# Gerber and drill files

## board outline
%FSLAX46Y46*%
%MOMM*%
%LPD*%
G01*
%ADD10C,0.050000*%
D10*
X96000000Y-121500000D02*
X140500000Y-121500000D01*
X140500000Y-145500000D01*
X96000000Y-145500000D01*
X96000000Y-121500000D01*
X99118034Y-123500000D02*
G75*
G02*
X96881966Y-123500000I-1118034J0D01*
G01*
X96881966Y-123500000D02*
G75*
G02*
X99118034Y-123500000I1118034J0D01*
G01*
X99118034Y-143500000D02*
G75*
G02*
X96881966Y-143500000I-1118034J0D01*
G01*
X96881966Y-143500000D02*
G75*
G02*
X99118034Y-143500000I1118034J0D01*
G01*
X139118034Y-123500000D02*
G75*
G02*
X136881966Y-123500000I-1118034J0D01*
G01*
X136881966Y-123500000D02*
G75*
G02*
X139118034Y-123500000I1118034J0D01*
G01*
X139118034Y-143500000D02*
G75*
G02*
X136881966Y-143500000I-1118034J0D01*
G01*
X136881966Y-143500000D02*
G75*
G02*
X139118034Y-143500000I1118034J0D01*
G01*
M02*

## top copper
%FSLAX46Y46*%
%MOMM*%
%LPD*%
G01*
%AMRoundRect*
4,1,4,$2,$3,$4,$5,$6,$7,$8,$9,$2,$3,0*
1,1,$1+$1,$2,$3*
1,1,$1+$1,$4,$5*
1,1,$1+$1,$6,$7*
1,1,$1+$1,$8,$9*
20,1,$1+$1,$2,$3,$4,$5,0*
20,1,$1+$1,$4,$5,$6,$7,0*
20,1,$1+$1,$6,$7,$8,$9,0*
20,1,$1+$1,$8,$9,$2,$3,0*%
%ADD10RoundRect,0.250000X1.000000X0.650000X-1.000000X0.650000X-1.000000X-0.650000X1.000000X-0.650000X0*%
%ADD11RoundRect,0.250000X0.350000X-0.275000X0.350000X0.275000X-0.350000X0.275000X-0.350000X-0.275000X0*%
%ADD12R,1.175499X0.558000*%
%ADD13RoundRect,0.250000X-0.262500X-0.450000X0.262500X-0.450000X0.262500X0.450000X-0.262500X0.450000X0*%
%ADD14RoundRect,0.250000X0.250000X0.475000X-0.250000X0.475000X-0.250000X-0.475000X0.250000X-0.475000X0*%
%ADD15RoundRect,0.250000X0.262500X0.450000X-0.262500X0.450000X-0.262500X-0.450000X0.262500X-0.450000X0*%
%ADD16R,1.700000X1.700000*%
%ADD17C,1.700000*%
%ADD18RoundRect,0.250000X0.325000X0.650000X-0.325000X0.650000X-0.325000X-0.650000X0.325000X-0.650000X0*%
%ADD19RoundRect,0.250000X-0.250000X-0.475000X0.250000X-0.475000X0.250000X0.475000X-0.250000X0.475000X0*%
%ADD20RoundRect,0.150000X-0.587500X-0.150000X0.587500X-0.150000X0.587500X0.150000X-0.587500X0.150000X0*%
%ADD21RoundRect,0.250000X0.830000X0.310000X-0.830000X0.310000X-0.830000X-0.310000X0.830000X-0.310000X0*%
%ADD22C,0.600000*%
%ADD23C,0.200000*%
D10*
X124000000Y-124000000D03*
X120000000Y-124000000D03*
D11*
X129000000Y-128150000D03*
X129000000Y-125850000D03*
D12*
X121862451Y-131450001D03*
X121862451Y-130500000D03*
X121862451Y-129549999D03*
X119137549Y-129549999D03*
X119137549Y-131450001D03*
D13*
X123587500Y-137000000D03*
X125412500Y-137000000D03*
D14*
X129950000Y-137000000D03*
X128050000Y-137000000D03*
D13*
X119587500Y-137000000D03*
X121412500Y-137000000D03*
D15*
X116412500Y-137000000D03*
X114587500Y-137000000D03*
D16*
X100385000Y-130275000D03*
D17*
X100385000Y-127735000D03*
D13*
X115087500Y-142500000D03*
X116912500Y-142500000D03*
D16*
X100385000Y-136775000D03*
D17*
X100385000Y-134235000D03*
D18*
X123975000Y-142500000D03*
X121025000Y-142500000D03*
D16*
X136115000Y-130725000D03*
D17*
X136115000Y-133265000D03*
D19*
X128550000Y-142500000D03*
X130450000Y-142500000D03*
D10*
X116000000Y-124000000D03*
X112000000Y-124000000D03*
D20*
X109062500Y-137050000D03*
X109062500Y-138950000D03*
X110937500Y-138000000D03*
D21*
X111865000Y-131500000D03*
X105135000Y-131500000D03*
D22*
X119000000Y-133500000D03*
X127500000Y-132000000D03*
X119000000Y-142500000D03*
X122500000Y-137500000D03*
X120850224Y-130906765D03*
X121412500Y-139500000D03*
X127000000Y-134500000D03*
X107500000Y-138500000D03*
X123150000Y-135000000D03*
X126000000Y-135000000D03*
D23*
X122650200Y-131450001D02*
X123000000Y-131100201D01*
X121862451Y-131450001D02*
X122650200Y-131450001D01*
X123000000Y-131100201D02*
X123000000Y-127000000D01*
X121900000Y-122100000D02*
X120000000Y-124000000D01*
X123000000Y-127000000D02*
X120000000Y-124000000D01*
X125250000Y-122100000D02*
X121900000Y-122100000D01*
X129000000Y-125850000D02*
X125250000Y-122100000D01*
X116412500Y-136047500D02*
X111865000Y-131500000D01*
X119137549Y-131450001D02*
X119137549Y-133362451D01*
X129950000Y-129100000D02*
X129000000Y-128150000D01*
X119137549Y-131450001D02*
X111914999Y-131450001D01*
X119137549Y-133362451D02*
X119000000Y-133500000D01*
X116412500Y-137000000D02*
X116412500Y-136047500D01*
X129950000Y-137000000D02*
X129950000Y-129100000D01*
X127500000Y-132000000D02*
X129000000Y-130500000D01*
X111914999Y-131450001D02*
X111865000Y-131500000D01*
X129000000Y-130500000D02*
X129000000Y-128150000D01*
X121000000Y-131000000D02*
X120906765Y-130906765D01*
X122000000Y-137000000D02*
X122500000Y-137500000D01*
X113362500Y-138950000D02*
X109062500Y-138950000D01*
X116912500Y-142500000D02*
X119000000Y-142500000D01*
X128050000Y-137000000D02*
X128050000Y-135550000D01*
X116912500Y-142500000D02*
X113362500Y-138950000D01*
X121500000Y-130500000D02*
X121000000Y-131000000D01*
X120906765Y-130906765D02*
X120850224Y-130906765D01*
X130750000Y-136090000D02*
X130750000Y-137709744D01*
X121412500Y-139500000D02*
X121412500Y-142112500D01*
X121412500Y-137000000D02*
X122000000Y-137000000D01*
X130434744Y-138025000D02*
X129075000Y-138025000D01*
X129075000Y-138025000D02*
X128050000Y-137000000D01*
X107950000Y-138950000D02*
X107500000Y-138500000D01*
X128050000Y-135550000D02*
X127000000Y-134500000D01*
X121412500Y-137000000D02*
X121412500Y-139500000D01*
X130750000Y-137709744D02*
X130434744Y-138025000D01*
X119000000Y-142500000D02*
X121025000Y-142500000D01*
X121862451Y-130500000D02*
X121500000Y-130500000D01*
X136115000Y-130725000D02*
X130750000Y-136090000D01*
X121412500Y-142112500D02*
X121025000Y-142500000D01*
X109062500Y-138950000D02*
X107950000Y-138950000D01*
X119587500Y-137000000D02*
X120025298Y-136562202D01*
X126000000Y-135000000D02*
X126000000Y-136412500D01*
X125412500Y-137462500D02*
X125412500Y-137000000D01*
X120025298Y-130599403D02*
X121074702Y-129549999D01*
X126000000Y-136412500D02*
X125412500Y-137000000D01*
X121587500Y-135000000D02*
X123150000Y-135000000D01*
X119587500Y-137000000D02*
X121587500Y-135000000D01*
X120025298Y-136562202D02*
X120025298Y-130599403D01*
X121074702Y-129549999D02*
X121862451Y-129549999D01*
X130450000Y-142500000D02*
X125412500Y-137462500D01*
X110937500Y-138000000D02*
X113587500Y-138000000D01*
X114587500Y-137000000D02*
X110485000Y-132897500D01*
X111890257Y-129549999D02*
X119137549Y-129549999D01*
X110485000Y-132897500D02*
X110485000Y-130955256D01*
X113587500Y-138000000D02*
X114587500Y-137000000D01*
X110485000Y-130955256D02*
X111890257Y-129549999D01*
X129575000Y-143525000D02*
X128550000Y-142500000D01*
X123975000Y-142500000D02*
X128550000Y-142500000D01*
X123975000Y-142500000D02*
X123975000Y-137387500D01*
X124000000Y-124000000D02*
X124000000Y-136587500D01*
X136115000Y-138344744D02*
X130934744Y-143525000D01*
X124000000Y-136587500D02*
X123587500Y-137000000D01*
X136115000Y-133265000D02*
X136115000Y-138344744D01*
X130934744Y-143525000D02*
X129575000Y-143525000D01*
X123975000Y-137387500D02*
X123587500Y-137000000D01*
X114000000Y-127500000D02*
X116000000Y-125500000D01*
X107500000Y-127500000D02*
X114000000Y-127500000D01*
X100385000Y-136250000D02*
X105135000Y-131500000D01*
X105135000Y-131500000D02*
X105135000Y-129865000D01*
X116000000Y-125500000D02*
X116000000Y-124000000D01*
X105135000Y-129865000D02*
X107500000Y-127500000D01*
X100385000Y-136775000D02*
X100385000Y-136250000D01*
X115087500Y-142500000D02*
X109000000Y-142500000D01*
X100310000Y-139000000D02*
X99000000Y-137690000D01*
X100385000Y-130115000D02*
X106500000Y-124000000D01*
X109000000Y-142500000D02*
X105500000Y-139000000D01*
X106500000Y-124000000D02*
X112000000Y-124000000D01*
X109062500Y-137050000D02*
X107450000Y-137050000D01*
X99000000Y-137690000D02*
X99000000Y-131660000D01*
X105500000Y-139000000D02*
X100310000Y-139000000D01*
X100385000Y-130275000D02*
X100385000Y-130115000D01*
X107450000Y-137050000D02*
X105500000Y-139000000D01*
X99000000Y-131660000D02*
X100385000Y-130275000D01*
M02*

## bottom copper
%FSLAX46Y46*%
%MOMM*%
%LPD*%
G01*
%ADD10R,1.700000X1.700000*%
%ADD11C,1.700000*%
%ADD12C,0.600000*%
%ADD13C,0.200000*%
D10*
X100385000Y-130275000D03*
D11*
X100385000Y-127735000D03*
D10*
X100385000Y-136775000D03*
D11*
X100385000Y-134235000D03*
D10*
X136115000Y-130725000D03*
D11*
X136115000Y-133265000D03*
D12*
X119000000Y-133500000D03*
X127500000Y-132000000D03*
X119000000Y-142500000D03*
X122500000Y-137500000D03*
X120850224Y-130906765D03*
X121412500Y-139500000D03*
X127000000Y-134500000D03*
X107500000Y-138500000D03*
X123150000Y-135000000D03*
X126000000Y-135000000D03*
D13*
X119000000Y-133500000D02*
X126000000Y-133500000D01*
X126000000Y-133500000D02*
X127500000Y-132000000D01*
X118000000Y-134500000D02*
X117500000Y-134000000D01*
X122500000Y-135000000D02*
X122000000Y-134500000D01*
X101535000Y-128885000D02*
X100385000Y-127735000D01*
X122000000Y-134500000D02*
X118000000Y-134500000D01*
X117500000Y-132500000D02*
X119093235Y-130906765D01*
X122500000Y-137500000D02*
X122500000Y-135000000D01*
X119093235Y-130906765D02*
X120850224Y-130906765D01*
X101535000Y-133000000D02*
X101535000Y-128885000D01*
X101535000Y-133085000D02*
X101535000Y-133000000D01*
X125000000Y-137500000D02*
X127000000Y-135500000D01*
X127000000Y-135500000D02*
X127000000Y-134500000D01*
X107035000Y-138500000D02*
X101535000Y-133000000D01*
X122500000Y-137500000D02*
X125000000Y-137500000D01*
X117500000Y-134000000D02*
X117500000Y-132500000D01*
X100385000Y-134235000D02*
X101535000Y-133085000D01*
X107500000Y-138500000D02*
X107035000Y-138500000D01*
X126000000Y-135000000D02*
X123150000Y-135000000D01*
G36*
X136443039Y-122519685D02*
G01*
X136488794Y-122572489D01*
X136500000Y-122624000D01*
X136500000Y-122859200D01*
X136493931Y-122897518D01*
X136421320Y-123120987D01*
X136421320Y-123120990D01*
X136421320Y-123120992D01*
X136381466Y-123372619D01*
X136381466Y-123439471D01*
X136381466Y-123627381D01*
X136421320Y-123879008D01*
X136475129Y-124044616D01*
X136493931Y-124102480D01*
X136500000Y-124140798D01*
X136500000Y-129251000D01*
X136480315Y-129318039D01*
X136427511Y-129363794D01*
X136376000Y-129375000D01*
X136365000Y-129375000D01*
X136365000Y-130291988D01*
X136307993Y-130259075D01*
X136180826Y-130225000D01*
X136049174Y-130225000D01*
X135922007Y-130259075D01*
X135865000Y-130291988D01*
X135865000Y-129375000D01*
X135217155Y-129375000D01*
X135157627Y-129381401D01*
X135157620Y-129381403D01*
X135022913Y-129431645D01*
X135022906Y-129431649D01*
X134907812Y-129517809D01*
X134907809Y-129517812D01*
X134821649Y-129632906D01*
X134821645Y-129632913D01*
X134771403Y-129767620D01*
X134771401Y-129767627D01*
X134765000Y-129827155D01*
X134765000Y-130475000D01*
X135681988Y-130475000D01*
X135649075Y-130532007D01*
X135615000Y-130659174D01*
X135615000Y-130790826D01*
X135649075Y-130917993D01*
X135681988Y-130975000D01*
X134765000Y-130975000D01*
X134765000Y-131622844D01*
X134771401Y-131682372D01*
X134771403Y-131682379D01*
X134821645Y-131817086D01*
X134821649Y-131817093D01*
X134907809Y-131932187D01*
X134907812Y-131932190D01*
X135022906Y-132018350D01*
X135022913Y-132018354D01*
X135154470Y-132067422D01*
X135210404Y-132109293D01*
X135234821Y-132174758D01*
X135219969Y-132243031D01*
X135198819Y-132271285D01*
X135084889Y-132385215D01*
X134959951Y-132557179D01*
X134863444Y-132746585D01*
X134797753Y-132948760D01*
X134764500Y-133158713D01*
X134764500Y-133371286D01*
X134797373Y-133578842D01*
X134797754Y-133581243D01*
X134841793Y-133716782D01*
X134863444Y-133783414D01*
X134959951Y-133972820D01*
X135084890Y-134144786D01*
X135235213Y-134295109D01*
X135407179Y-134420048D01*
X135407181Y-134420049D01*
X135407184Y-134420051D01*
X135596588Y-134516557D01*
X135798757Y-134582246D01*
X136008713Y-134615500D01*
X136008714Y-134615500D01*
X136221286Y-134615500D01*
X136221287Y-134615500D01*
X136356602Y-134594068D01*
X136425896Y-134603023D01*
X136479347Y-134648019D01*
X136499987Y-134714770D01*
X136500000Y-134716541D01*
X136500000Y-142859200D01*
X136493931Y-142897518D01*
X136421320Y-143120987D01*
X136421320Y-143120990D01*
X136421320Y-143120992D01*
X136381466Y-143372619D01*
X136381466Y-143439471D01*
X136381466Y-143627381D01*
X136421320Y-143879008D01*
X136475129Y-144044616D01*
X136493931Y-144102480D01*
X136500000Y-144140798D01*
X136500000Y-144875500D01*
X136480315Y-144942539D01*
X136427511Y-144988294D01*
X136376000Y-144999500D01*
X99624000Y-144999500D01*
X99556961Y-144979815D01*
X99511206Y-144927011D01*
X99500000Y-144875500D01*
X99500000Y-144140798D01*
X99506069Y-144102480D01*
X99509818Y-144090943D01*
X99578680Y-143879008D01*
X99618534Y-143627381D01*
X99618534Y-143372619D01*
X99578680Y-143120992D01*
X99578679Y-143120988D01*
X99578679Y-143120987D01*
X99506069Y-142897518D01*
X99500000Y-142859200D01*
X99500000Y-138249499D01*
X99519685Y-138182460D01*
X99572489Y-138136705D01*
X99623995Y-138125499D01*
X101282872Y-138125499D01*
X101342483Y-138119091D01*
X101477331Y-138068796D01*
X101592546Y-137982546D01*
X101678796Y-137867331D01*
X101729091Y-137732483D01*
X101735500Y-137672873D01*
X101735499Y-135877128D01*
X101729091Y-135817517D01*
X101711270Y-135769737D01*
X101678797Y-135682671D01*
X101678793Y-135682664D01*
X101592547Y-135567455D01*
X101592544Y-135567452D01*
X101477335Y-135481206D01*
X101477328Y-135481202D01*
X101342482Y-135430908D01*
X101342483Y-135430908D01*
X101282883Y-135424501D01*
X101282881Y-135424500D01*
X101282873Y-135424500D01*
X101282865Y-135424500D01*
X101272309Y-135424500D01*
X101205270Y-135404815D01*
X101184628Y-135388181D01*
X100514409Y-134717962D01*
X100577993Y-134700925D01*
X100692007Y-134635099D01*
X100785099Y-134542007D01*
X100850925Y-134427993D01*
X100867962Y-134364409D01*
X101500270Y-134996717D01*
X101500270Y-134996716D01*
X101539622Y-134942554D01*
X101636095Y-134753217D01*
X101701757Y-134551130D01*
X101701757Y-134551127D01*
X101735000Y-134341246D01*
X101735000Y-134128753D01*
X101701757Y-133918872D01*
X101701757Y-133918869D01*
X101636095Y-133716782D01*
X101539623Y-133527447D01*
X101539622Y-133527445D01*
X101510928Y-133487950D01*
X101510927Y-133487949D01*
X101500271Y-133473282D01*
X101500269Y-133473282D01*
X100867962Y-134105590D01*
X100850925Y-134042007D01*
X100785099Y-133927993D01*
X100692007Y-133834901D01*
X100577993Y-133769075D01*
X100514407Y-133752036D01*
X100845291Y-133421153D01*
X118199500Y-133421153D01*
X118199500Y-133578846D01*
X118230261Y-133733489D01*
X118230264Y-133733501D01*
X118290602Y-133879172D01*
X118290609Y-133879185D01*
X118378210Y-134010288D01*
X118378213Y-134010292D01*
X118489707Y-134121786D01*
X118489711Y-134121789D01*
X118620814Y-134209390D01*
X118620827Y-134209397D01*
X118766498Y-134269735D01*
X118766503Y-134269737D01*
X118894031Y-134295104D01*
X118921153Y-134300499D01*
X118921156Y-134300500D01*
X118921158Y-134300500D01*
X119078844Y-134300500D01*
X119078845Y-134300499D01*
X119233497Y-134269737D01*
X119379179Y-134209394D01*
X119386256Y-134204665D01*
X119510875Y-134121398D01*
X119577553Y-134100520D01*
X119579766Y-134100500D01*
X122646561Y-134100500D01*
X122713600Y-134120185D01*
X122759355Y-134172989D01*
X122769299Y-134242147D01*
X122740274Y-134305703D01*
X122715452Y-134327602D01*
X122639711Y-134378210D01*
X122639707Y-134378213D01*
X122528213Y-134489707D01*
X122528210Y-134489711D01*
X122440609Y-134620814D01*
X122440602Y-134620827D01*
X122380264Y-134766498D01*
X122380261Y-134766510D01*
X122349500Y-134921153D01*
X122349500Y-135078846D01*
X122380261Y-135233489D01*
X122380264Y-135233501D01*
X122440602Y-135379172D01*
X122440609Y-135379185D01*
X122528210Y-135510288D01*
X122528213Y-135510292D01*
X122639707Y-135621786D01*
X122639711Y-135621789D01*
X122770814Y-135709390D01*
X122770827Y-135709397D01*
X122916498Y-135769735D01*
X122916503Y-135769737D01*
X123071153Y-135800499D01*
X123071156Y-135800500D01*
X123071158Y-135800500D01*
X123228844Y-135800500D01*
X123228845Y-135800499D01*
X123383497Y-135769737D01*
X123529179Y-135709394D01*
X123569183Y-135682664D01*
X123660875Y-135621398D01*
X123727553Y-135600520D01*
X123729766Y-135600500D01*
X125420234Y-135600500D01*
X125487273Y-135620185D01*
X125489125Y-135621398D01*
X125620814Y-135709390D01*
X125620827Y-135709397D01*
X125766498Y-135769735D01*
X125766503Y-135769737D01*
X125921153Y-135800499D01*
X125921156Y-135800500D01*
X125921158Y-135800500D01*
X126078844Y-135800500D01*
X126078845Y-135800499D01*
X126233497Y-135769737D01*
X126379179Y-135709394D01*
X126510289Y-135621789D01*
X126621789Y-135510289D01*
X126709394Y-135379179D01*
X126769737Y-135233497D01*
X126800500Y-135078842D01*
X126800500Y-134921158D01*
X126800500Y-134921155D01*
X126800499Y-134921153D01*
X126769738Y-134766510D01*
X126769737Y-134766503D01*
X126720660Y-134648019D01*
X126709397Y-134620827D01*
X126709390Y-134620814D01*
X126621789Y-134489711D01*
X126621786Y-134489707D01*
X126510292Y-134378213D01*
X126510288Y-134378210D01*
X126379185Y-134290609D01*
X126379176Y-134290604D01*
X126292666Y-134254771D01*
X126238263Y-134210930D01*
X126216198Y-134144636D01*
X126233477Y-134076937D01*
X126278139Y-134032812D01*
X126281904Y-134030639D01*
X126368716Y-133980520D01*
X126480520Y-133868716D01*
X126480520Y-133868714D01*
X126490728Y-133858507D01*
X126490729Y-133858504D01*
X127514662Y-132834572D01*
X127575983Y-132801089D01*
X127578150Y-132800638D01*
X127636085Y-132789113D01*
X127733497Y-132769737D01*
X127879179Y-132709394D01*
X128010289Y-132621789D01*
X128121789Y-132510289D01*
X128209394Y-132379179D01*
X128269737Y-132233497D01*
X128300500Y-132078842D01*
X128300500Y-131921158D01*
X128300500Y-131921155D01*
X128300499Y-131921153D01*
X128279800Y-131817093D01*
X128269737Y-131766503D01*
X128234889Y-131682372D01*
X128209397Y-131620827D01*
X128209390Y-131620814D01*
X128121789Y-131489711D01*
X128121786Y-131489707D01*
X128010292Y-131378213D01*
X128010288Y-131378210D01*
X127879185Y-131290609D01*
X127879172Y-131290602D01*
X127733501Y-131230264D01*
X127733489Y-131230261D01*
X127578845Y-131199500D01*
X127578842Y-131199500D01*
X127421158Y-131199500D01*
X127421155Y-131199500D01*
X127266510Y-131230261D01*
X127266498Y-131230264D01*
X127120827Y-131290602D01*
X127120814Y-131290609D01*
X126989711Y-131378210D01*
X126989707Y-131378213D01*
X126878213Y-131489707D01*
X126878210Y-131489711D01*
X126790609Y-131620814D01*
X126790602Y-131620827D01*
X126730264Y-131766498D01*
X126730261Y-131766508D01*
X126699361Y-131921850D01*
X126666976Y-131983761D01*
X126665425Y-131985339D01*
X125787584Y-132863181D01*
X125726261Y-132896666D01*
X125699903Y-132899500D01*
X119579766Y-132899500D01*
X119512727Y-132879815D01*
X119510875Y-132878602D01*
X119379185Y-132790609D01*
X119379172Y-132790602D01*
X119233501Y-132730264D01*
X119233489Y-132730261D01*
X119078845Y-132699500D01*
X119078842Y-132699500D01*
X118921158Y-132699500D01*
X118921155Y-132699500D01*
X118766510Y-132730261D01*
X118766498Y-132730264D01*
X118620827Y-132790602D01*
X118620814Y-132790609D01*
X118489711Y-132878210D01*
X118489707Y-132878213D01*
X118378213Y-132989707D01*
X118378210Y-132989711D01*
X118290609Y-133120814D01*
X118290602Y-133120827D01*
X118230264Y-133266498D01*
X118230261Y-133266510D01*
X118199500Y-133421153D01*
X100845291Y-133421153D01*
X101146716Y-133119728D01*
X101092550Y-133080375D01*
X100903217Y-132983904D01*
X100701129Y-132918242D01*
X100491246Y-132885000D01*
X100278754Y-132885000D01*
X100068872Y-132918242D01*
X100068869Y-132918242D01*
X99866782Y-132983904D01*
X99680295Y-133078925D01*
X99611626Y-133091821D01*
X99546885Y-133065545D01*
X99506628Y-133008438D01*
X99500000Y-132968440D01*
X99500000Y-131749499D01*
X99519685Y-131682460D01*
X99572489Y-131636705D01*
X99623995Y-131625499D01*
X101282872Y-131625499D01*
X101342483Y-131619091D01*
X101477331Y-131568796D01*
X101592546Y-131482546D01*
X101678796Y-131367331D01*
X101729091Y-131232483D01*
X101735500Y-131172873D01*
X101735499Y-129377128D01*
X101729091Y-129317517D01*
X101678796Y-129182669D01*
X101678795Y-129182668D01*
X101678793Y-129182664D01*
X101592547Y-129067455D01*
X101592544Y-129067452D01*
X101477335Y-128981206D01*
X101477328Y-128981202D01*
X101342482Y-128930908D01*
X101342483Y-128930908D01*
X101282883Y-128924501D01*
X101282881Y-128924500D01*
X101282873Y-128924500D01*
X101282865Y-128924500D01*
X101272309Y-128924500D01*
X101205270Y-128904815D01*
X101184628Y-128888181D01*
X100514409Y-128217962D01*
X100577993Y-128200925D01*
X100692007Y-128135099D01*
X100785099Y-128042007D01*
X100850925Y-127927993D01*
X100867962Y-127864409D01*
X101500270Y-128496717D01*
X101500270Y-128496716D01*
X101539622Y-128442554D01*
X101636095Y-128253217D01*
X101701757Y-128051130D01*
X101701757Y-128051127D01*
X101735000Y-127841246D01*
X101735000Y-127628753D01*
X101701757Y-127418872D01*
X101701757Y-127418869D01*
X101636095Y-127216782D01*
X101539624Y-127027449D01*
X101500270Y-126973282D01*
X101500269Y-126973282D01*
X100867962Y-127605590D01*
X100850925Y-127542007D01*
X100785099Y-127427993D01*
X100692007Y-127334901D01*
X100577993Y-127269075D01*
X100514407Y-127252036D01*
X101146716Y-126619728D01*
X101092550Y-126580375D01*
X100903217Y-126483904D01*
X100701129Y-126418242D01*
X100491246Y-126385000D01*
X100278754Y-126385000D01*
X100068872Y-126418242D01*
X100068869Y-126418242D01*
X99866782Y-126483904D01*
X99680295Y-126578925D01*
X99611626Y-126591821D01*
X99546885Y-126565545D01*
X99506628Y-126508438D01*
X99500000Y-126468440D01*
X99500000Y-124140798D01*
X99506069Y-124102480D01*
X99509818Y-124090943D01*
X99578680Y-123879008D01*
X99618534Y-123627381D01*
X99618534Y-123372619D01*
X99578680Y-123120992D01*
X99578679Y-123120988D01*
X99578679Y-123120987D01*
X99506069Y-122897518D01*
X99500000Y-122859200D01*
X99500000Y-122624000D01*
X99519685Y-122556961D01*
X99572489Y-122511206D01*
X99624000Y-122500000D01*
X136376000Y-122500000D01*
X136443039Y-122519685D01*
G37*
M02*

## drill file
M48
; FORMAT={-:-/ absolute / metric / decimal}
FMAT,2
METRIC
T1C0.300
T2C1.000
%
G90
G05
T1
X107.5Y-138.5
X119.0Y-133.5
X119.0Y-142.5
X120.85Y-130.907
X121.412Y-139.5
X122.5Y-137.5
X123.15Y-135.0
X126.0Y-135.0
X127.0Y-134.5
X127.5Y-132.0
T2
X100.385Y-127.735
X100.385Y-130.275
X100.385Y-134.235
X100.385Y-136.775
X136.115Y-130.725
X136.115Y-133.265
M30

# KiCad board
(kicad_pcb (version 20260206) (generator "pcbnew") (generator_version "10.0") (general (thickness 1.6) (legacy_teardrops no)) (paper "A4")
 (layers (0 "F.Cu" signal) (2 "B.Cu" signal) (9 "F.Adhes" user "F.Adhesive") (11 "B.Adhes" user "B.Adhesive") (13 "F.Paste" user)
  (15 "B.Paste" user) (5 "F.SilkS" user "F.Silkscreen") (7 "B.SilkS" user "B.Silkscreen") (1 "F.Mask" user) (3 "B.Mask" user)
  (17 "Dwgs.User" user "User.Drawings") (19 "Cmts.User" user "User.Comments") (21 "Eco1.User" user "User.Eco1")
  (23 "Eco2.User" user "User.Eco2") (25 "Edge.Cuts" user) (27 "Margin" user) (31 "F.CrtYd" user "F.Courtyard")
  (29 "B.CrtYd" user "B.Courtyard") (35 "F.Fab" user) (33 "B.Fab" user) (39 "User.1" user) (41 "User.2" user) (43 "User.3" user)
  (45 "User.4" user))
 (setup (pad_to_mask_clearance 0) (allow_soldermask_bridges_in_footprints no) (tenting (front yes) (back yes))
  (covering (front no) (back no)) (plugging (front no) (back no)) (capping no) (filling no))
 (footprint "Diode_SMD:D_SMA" (layer "F.Cu") (at 122 124 180)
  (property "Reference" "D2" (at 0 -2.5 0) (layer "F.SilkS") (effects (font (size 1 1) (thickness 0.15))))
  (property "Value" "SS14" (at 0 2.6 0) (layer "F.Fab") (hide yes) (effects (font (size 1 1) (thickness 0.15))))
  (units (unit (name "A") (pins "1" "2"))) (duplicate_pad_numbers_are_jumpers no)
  (pad "1" smd roundrect (at -2 0 180) (size 2.5 1.8) (layers "F.Cu" "F.Mask" "F.Paste") (roundrect_rratio 0.1388888889) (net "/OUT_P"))
  (pad "2" smd roundrect (at 2 0 180) (size 2.5 1.8) (layers "F.Cu" "F.Mask" "F.Paste") (roundrect_rratio 0.1388888889) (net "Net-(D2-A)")))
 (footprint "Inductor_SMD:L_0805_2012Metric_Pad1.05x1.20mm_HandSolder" (layer "F.Cu") (at 129 127 90)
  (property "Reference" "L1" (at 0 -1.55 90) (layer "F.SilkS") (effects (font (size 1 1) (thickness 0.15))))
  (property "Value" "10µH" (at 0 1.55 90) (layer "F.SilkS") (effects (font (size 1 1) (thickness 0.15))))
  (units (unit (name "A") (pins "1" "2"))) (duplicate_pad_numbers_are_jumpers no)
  (pad "1" smd roundrect (at -1.15 0 90) (size 1.05 1.2) (layers "F.Cu" "F.Mask" "F.Paste") (roundrect_rratio 0.238095)
   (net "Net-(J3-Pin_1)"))
  (pad "2" smd roundrect (at 1.15 0 90) (size 1.05 1.2) (layers "F.Cu" "F.Mask" "F.Paste") (roundrect_rratio 0.238095) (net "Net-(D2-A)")))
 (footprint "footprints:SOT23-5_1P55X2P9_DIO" (layer "F.Cu") (at 120.5 130.5 180)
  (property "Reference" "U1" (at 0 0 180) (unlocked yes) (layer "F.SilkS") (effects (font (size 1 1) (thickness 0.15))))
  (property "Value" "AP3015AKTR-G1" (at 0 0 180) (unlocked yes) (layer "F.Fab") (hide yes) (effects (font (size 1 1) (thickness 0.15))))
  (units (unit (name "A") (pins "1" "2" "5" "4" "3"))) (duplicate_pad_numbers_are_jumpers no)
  (pad "1" smd rect (at -1.362451 -0.950001 180) (size 1.175499 0.558) (layers "F.Cu" "F.Mask" "F.Paste") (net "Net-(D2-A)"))
  (pad "2" smd rect (at -1.362451 0 180) (size 1.175499 0.558) (layers "F.Cu" "F.Mask" "F.Paste") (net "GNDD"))
  (pad "3" smd rect (at -1.362451 0.950001 180) (size 1.175499 0.558) (layers "F.Cu" "F.Mask" "F.Paste") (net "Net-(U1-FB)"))
  (pad "4" smd rect (at 1.362451 0.950001 180) (size 1.175499 0.558) (layers "F.Cu" "F.Mask" "F.Paste") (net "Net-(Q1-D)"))
  (pad "5" smd rect (at 1.362451 -0.950001 180) (size 1.175499 0.558) (layers "F.Cu" "F.Mask" "F.Paste") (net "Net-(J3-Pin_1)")))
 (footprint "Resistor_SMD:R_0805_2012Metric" (layer "F.Cu") (at 124.5 137)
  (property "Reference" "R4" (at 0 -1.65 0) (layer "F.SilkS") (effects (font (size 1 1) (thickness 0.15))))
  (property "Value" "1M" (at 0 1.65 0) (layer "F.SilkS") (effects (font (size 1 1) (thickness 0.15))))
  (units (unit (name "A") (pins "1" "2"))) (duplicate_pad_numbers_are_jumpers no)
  (pad "1" smd roundrect (at -0.9125 0) (size 1.025 1.4) (layers "F.Cu" "F.Mask" "F.Paste") (roundrect_rratio 0.243902) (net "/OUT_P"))
  (pad "2" smd roundrect (at 0.9125 0) (size 1.025 1.4) (layers "F.Cu" "F.Mask" "F.Paste") (roundrect_rratio 0.243902) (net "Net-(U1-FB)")))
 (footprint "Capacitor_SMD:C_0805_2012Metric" (layer "F.Cu") (at 129 137 180)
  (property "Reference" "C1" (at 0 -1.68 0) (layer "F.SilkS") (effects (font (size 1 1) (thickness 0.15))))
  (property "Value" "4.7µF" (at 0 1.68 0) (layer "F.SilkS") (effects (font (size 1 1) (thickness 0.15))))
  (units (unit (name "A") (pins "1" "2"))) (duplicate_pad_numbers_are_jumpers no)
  (pad "1" smd roundrect (at -0.95 0 180) (size 1 1.45) (layers "F.Cu" "F.Mask" "F.Paste") (roundrect_rratio 0.25) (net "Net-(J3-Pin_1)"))
  (pad "2" smd roundrect (at 0.95 0 180) (size 1 1.45) (layers "F.Cu" "F.Mask" "F.Paste") (roundrect_rratio 0.25) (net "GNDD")))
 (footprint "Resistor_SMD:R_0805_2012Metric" (layer "F.Cu") (at 120.5 137)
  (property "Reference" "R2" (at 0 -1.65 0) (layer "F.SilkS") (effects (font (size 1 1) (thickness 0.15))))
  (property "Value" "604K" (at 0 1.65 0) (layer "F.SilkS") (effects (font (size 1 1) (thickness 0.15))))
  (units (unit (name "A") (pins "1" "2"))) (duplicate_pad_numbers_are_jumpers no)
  (pad "1" smd roundrect (at -0.9125 0) (size 1.025 1.4) (layers "F.Cu" "F.Mask" "F.Paste") (roundrect_rratio 0.243902) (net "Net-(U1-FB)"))
  (pad "2" smd roundrect (at 0.9125 0) (size 1.025 1.4) (layers "F.Cu" "F.Mask" "F.Paste") (roundrect_rratio 0.243902) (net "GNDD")))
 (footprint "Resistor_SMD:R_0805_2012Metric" (layer "F.Cu") (at 115.5 137 180)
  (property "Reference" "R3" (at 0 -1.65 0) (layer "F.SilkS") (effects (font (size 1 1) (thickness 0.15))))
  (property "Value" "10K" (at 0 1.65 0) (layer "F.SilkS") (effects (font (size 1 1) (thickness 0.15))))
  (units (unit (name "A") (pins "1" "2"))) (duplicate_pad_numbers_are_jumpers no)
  (pad "1" smd roundrect (at -0.9125 0 180) (size 1.025 1.4) (layers "F.Cu" "F.Mask" "F.Paste") (roundrect_rratio 0.243902)
   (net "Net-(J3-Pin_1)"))
  (pad "2" smd roundrect (at 0.9125 0 180) (size 1.025 1.4) (layers "F.Cu" "F.Mask" "F.Paste") (roundrect_rratio 0.243902)
   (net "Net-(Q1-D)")))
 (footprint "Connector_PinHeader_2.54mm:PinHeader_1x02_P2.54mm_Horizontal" (layer "F.Cu") (at 100.385 130.275 180)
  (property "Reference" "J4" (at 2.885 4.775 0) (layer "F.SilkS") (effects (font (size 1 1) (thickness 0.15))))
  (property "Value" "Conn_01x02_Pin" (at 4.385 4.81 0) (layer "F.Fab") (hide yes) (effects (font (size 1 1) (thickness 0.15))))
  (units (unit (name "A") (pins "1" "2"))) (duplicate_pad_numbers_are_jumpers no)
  (pad "1" thru_hole rect (at 0 0 180) (size 1.7 1.7) (drill 1) (layers "*.Cu" "*.Mask") (remove_unused_layers no) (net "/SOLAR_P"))
  (pad "2" thru_hole circle (at 0 2.54 180) (size 1.7 1.7) (drill 1) (layers "*.Cu" "*.Mask") (remove_unused_layers no) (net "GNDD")))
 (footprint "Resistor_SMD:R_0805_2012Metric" (layer "F.Cu") (at 116 142.5)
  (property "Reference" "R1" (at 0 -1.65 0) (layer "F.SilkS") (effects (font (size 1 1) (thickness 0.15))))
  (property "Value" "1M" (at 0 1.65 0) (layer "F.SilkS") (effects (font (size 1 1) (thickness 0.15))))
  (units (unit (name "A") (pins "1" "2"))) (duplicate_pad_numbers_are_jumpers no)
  (pad "1" smd roundrect (at -0.9125 0) (size 1.025 1.4) (layers "F.Cu" "F.Mask" "F.Paste") (roundrect_rratio 0.243902) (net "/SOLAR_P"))
  (pad "2" smd roundrect (at 0.9125 0) (size 1.025 1.4) (layers "F.Cu" "F.Mask" "F.Paste") (roundrect_rratio 0.243902) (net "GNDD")))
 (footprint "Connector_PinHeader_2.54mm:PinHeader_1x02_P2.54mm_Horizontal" (layer "F.Cu") (at 100.385 136.775 180)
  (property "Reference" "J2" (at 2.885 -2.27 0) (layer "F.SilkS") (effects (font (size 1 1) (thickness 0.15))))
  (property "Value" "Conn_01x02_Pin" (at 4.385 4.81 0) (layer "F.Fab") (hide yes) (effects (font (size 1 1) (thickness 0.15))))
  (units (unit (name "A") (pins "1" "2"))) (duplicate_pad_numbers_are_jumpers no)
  (pad "1" thru_hole rect (at 0 0 180) (size 1.7 1.7) (drill 1) (layers "*.Cu" "*.Mask") (remove_unused_layers no) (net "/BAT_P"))
  (pad "2" thru_hole circle (at 0 2.54 180) (size 1.7 1.7) (drill 1) (layers "*.Cu" "*.Mask") (remove_unused_layers no) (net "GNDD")))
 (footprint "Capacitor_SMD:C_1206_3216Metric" (layer "F.Cu") (at 122.5 142.5 180)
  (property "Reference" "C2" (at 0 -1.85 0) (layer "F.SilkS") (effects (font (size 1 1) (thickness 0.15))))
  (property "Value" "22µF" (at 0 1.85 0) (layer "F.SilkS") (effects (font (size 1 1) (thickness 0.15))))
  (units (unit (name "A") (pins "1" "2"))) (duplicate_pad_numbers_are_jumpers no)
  (pad "1" smd roundrect (at -1.475 0 180) (size 1.15 1.8) (layers "F.Cu" "F.Mask" "F.Paste") (roundrect_rratio 0.217391) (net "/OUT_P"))
  (pad "2" smd roundrect (at 1.475 0 180) (size 1.15 1.8) (layers "F.Cu" "F.Mask" "F.Paste") (roundrect_rratio 0.217391) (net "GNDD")))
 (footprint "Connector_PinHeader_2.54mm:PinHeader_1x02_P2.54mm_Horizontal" (layer "F.Cu") (at 136.115 130.725)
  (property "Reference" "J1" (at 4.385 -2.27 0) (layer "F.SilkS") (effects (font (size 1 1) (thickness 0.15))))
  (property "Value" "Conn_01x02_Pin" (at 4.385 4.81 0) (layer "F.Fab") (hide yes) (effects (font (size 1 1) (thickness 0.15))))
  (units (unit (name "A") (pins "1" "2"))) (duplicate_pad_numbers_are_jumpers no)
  (pad "1" thru_hole rect (at 0 0) (size 1.7 1.7) (drill 1) (layers "*.Cu" "*.Mask") (remove_unused_layers no) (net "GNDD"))
  (pad "2" thru_hole circle (at 0 2.54) (size 1.7 1.7) (drill 1) (layers "*.Cu" "*.Mask") (remove_unused_layers no) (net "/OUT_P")))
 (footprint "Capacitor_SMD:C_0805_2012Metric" (layer "F.Cu") (at 129.5 142.5)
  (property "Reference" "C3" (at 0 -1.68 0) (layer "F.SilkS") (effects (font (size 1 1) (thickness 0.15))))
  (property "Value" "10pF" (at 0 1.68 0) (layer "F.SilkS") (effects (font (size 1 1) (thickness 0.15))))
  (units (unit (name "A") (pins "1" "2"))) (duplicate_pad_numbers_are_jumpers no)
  (pad "1" smd roundrect (at -0.95 0) (size 1 1.45) (layers "F.Cu" "F.Mask" "F.Paste") (roundrect_rratio 0.25) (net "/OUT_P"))
  (pad "2" smd roundrect (at 0.95 0) (size 1 1.45) (layers "F.Cu" "F.Mask" "F.Paste") (roundrect_rratio 0.25) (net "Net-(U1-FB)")))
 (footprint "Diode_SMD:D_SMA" (layer "F.Cu") (at 114 124 180)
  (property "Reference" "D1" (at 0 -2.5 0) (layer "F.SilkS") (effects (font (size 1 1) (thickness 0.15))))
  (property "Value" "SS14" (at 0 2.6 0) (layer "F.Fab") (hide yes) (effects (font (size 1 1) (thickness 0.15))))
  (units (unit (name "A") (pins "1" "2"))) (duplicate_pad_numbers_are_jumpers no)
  (pad "1" smd roundrect (at -2 0 180) (size 2.5 1.8) (layers "F.Cu" "F.Mask" "F.Paste") (roundrect_rratio 0.1388888889) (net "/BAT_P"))
  (pad "2" smd roundrect (at 2 0 180) (size 2.5 1.8) (layers "F.Cu" "F.Mask" "F.Paste") (roundrect_rratio 0.1388888889) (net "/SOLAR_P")))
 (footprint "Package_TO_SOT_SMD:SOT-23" (layer "F.Cu") (at 110 138)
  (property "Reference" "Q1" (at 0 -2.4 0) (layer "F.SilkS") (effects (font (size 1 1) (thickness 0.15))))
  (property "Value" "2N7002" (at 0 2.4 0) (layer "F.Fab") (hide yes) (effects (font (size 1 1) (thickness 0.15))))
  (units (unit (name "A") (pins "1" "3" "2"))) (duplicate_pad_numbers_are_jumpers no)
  (pad "1" smd roundrect (at -0.9375 -0.95) (size 1.475 0.6) (layers "F.Cu" "F.Mask" "F.Paste") (roundrect_rratio 0.25) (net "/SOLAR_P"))
  (pad "2" smd roundrect (at -0.9375 0.95) (size 1.475 0.6) (layers "F.Cu" "F.Mask" "F.Paste") (roundrect_rratio 0.25) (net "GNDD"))
  (pad "3" smd roundrect (at 0.9375 0) (size 1.475 0.6) (layers "F.Cu" "F.Mask" "F.Paste") (roundrect_rratio 0.25) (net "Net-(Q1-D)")))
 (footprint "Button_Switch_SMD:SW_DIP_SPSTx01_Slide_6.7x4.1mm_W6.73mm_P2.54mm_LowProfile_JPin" (layer "F.Cu") (at 108.5 131.5 180)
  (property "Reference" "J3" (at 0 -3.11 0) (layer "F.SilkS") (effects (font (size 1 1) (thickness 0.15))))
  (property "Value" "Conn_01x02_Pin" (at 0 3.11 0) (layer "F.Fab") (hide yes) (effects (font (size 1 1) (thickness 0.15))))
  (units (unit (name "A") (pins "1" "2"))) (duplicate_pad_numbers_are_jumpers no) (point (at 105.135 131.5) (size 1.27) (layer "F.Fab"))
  (pad "1" smd roundrect (at -3.365 0 180) (size 2.16 1.12) (layers "F.Cu" "F.Mask" "F.Paste") (roundrect_rratio 0.223214)
   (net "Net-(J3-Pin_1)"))
  (pad "2" smd roundrect (at 3.365 0 180) (size 2.16 1.12) (layers "F.Cu" "F.Mask" "F.Paste") (roundrect_rratio 0.223214) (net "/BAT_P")))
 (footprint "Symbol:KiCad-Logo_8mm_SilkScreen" (layer "B.Cu") (at 117.5 129.5 180)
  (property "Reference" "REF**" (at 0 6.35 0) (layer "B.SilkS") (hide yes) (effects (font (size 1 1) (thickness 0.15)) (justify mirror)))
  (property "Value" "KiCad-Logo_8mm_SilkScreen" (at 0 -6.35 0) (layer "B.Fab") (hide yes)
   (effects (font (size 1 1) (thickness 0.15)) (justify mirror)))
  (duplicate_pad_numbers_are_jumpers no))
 (gr_rect (start 96 121.5) (end 140.5 145.5) (stroke (width 0.05) (type default)) (fill no) (layer "Edge.Cuts"))
 (gr_circle (center 98 123.5) (end 97 123) (stroke (width 0.05) (type default)) (fill no) (layer "Edge.Cuts"))
 (gr_circle (center 98 143.5) (end 97 143) (stroke (width 0.05) (type default)) (fill no) (layer "Edge.Cuts"))
 (gr_circle (center 138 123.5) (end 137 123) (stroke (width 0.05) (type default)) (fill no) (layer "Edge.Cuts"))
 (gr_circle (center 138 143.5) (end 137 143) (stroke (width 0.05) (type default)) (fill no) (layer "Edge.Cuts"))
 (segment (start 122.6502 131.450001) (end 123 131.100201) (width 0.2) (layer "F.Cu") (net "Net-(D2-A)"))
 (segment (start 121.862451 131.450001) (end 122.6502 131.450001) (width 0.2) (layer "F.Cu") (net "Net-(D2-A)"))
 (segment (start 123 131.100201) (end 123 127) (width 0.2) (layer "F.Cu") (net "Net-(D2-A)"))
 (segment (start 121.9 122.1) (end 120 124) (width 0.2) (layer "F.Cu") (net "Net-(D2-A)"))
 (segment (start 123 127) (end 120 124) (width 0.2) (layer "F.Cu") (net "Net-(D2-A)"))
 (segment (start 125.25 122.1) (end 121.9 122.1) (width 0.2) (layer "F.Cu") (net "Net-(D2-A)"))
 (segment (start 129 125.85) (end 125.25 122.1) (width 0.2) (layer "F.Cu") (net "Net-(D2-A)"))
 (segment (start 116.4125 136.0475) (end 111.865 131.5) (width 0.2) (layer "F.Cu") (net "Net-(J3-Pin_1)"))
 (segment (start 119.137549 131.450001) (end 119.137549 133.362451) (width 0.2) (layer "F.Cu") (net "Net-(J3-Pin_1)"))
 (segment (start 129.95 129.1) (end 129 128.15) (width 0.2) (layer "F.Cu") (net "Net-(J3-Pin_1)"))
 (segment (start 119.137549 131.450001) (end 111.914999 131.450001) (width 0.2) (layer "F.Cu") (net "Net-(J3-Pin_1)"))
 (segment (start 119.137549 133.362451) (end 119 133.5) (width 0.2) (layer "F.Cu") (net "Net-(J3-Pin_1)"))
 (segment (start 116.4125 137) (end 116.4125 136.0475) (width 0.2) (layer "F.Cu") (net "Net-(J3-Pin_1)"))
 (segment (start 129.95 137) (end 129.95 129.1) (width 0.2) (layer "F.Cu") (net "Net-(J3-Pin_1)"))
 (segment (start 127.5 132) (end 129 130.5) (width 0.2) (layer "F.Cu") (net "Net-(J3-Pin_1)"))
 (segment (start 111.914999 131.450001) (end 111.865 131.5) (width 0.2) (layer "F.Cu") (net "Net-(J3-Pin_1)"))
 (segment (start 129 130.5) (end 129 128.15) (width 0.2) (layer "F.Cu") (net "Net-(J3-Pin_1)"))
 (via (at 119 133.5) (size 0.6) (drill 0.3) (layers "F.Cu" "B.Cu") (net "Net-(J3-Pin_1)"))
 (via (at 127.5 132) (size 0.6) (drill 0.3) (layers "F.Cu" "B.Cu") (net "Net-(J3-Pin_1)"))
 (segment (start 119 133.5) (end 126 133.5) (width 0.2) (layer "B.Cu") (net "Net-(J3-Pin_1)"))
 (segment (start 126 133.5) (end 127.5 132) (width 0.2) (layer "B.Cu") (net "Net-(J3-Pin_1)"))
 (segment (start 121 131) (end 120.906765 130.906765) (width 0.2) (layer "F.Cu") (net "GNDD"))
 (segment (start 122 137) (end 122.5 137.5) (width 0.2) (layer "F.Cu") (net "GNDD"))
 (segment (start 113.3625 138.95) (end 109.0625 138.95) (width 0.2) (layer "F.Cu") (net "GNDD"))
 (segment (start 116.9125 142.5) (end 119 142.5) (width 0.2) (layer "F.Cu") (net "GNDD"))
 (segment (start 128.05 137) (end 128.05 135.55) (width 0.2) (layer "F.Cu") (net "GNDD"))
 (segment (start 116.9125 142.5) (end 113.3625 138.95) (width 0.2) (layer "F.Cu") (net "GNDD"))
 (segment (start 121.5 130.5) (end 121 131) (width 0.2) (layer "F.Cu") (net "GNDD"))
 (segment (start 120.906765 130.906765) (end 120.850224 130.906765) (width 0.2) (layer "F.Cu") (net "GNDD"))
 (segment (start 130.75 136.09) (end 130.75 137.709744) (width 0.2) (layer "F.Cu") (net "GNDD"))
 (segment (start 121.4125 139.5) (end 121.4125 142.1125) (width 0.2) (layer "F.Cu") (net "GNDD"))
 (segment (start 121.4125 137) (end 122 137) (width 0.2) (layer "F.Cu") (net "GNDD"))
 (segment (start 130.434744 138.025) (end 129.075 138.025) (width 0.2) (layer "F.Cu") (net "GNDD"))
 (segment (start 129.075 138.025) (end 128.05 137) (width 0.2) (layer "F.Cu") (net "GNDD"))
 (segment (start 107.95 138.95) (end 107.5 138.5) (width 0.2) (layer "F.Cu") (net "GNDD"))
 (segment (start 128.05 135.55) (end 127 134.5) (width 0.2) (layer "F.Cu") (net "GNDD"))
 (segment (start 121.4125 137) (end 121.4125 139.5) (width 0.2) (layer "F.Cu") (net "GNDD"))
 (segment (start 130.75 137.709744) (end 130.434744 138.025) (width 0.2) (layer "F.Cu") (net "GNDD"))
 (segment (start 119 142.5) (end 121.025 142.5) (width 0.2) (layer "F.Cu") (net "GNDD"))
 (segment (start 121.862451 130.5) (end 121.5 130.5) (width 0.2) (layer "F.Cu") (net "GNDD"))
 (segment (start 136.115 130.725) (end 130.75 136.09) (width 0.2) (layer "F.Cu") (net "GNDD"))
 (segment (start 121.4125 142.1125) (end 121.025 142.5) (width 0.2) (layer "F.Cu") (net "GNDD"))
 (segment (start 109.0625 138.95) (end 107.95 138.95) (width 0.2) (layer "F.Cu") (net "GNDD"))
 (via (at 119 142.5) (size 0.6) (drill 0.3) (layers "F.Cu" "B.Cu") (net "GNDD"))
 (via (at 122.5 137.5) (size 0.6) (drill 0.3) (layers "F.Cu" "B.Cu") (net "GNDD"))
 (via (at 120.850224 130.906765) (size 0.6) (drill 0.3) (layers "F.Cu" "B.Cu") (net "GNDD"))
 (via (at 121.4125 139.5) (size 0.6) (drill 0.3) (layers "F.Cu" "B.Cu") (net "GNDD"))
 (via (at 127 134.5) (size 0.6) (drill 0.3) (layers "F.Cu" "B.Cu") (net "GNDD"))
 (via (at 107.5 138.5) (size 0.6) (drill 0.3) (layers "F.Cu" "B.Cu") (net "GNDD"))
 (segment (start 118 134.5) (end 117.5 134) (width 0.2) (layer "B.Cu") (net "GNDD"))
 (segment (start 122.5 135) (end 122 134.5) (width 0.2) (layer "B.Cu") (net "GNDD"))
 (segment (start 101.535 128.885) (end 100.385 127.735) (width 0.2) (layer "B.Cu") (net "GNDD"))
 (segment (start 122 134.5) (end 118 134.5) (width 0.2) (layer "B.Cu") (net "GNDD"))
 (segment (start 117.5 132.5) (end 119.093235 130.906765) (width 0.2) (layer "B.Cu") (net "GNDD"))
 (segment (start 122.5 137.5) (end 122.5 135) (width 0.2) (layer "B.Cu") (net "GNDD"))
 (segment (start 119.093235 130.906765) (end 120.850224 130.906765) (width 0.2) (layer "B.Cu") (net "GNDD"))
 (segment (start 101.535 133) (end 101.535 128.885) (width 0.2) (layer "B.Cu") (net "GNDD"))
 (segment (start 101.535 133.085) (end 101.535 133) (width 0.2) (layer "B.Cu") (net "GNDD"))
 (segment (start 125 137.5) (end 127 135.5) (width 0.2) (layer "B.Cu") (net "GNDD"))
 (segment (start 127 135.5) (end 127 134.5) (width 0.2) (layer "B.Cu") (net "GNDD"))
 (segment (start 107.035 138.5) (end 101.535 133) (width 0.2) (layer "B.Cu") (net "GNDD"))
 (segment (start 122.5 137.5) (end 125 137.5) (width 0.2) (layer "B.Cu") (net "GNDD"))
 (segment (start 117.5 134) (end 117.5 132.5) (width 0.2) (layer "B.Cu") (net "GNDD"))
 (segment (start 100.385 134.235) (end 101.535 133.085) (width 0.2) (layer "B.Cu") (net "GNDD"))
 (segment (start 107.5 138.5) (end 107.035 138.5) (width 0.2) (layer "B.Cu") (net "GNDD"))
 (segment (start 119.5875 137) (end 120.025298 136.562202) (width 0.2) (layer "F.Cu") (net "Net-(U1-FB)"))
 (segment (start 126 135) (end 126 136.4125) (width 0.2) (layer "F.Cu") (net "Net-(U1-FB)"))
 (segment (start 125.4125 137.4625) (end 125.4125 137) (width 0.2) (layer "F.Cu") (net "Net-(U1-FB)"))
 (segment (start 120.025298 130.599403) (end 121.074702 129.549999) (width 0.2) (layer "F.Cu") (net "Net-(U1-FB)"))
 (segment (start 126 136.4125) (end 125.4125 137) (width 0.2) (layer "F.Cu") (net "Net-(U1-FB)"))
 (segment (start 121.5875 135) (end 123.15 135) (width 0.2) (layer "F.Cu") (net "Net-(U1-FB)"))
 (segment (start 119.5875 137) (end 121.5875 135) (width 0.2) (layer "F.Cu") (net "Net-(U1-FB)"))
 (segment (start 120.025298 136.562202) (end 120.025298 130.599403) (width 0.2) (layer "F.Cu") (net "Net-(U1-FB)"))
 (segment (start 121.074702 129.549999) (end 121.862451 129.549999) (width 0.2) (layer "F.Cu") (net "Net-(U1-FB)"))
 (segment (start 130.45 142.5) (end 125.4125 137.4625) (width 0.2) (layer "F.Cu") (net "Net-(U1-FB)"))
 (via (at 123.15 135) (size 0.6) (drill 0.3) (layers "F.Cu" "B.Cu") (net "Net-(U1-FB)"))
 (via (at 126 135) (size 0.6) (drill 0.3) (layers "F.Cu" "B.Cu") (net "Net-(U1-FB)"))
 (segment (start 126 135) (end 123.15 135) (width 0.2) (layer "B.Cu") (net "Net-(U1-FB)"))
 (segment (start 110.9375 138) (end 113.5875 138) (width 0.2) (layer "F.Cu") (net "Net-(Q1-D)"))
 (segment (start 114.5875 137) (end 110.485 132.8975) (width 0.2) (layer "F.Cu") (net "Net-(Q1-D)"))
 (segment (start 111.890257 129.549999) (end 119.137549 129.549999) (width 0.2) (layer "F.Cu") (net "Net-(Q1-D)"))
 (segment (start 110.485 132.8975) (end 110.485 130.955256) (width 0.2) (layer "F.Cu") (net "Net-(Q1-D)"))
 (segment (start 113.5875 138) (end 114.5875 137) (width 0.2) (layer "F.Cu") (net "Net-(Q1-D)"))
 (segment (start 110.485 130.955256) (end 111.890257 129.549999) (width 0.2) (layer "F.Cu") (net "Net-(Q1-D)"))
 (segment (start 129.575 143.525) (end 128.55 142.5) (width 0.2) (layer "F.Cu") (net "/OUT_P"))
 (segment (start 123.975 142.5) (end 128.55 142.5) (width 0.2) (layer "F.Cu") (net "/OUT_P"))
 (segment (start 123.975 142.5) (end 123.975 137.3875) (width 0.2) (layer "F.Cu") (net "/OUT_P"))
 (segment (start 124 124) (end 124 136.5875) (width 0.2) (layer "F.Cu") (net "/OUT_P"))
 (segment (start 136.115 138.344744) (end 130.934744 143.525) (width 0.2) (layer "F.Cu") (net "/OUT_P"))
 (segment (start 124 136.5875) (end 123.5875 137) (width 0.2) (layer "F.Cu") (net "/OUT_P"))
 (segment (start 136.115 133.265) (end 136.115 138.344744) (width 0.2) (layer "F.Cu") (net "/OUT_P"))
 (segment (start 130.934744 143.525) (end 129.575 143.525) (width 0.2) (layer "F.Cu") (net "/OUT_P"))
 (segment (start 123.975 137.3875) (end 123.5875 137) (width 0.2) (layer "F.Cu") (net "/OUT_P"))
 (segment (start 114 127.5) (end 116 125.5) (width 0.2) (layer "F.Cu") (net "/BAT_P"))
 (segment (start 107.5 127.5) (end 114 127.5) (width 0.2) (layer "F.Cu") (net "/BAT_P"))
 (segment (start 100.385 136.25) (end 105.135 131.5) (width 0.2) (layer "F.Cu") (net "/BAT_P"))
 (segment (start 105.135 131.5) (end 105.135 129.865) (width 0.2) (layer "F.Cu") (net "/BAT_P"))
 (segment (start 116 125.5) (end 116 124) (width 0.2) (layer "F.Cu") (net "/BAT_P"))
 (segment (start 105.135 129.865) (end 107.5 127.5) (width 0.2) (layer "F.Cu") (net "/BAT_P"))
 (segment (start 100.385 136.775) (end 100.385 136.25) (width 0.2) (layer "F.Cu") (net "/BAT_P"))
 (segment (start 115.0875 142.5) (end 109 142.5) (width 0.2) (layer "F.Cu") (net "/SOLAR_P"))
 (segment (start 100.31 139) (end 99 137.69) (width 0.2) (layer "F.Cu") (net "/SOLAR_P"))
 (segment (start 100.385 130.115) (end 106.5 124) (width 0.2) (layer "F.Cu") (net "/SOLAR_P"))
 (segment (start 109 142.5) (end 105.5 139) (width 0.2) (layer "F.Cu") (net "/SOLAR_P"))
 (segment (start 106.5 124) (end 112 124) (width 0.2) (layer "F.Cu") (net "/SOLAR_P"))
 (segment (start 109.0625 137.05) (end 107.45 137.05) (width 0.2) (layer "F.Cu") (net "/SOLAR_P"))
 (segment (start 99 137.69) (end 99 131.66) (width 0.2) (layer "F.Cu") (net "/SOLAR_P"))
 (segment (start 105.5 139) (end 100.31 139) (width 0.2) (layer "F.Cu") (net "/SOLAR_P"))
 (segment (start 100.385 130.275) (end 100.385 130.115) (width 0.2) (layer "F.Cu") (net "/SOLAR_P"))
 (segment (start 107.45 137.05) (end 105.5 139) (width 0.2) (layer "F.Cu") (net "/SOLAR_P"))
 (segment (start 99 131.66) (end 100.385 130.275) (width 0.2) (layer "F.Cu") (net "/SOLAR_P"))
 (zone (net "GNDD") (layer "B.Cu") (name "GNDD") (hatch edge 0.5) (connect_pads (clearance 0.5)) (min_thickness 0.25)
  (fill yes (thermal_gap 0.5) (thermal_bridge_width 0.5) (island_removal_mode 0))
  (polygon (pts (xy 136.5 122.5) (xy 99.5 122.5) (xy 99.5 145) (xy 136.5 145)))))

